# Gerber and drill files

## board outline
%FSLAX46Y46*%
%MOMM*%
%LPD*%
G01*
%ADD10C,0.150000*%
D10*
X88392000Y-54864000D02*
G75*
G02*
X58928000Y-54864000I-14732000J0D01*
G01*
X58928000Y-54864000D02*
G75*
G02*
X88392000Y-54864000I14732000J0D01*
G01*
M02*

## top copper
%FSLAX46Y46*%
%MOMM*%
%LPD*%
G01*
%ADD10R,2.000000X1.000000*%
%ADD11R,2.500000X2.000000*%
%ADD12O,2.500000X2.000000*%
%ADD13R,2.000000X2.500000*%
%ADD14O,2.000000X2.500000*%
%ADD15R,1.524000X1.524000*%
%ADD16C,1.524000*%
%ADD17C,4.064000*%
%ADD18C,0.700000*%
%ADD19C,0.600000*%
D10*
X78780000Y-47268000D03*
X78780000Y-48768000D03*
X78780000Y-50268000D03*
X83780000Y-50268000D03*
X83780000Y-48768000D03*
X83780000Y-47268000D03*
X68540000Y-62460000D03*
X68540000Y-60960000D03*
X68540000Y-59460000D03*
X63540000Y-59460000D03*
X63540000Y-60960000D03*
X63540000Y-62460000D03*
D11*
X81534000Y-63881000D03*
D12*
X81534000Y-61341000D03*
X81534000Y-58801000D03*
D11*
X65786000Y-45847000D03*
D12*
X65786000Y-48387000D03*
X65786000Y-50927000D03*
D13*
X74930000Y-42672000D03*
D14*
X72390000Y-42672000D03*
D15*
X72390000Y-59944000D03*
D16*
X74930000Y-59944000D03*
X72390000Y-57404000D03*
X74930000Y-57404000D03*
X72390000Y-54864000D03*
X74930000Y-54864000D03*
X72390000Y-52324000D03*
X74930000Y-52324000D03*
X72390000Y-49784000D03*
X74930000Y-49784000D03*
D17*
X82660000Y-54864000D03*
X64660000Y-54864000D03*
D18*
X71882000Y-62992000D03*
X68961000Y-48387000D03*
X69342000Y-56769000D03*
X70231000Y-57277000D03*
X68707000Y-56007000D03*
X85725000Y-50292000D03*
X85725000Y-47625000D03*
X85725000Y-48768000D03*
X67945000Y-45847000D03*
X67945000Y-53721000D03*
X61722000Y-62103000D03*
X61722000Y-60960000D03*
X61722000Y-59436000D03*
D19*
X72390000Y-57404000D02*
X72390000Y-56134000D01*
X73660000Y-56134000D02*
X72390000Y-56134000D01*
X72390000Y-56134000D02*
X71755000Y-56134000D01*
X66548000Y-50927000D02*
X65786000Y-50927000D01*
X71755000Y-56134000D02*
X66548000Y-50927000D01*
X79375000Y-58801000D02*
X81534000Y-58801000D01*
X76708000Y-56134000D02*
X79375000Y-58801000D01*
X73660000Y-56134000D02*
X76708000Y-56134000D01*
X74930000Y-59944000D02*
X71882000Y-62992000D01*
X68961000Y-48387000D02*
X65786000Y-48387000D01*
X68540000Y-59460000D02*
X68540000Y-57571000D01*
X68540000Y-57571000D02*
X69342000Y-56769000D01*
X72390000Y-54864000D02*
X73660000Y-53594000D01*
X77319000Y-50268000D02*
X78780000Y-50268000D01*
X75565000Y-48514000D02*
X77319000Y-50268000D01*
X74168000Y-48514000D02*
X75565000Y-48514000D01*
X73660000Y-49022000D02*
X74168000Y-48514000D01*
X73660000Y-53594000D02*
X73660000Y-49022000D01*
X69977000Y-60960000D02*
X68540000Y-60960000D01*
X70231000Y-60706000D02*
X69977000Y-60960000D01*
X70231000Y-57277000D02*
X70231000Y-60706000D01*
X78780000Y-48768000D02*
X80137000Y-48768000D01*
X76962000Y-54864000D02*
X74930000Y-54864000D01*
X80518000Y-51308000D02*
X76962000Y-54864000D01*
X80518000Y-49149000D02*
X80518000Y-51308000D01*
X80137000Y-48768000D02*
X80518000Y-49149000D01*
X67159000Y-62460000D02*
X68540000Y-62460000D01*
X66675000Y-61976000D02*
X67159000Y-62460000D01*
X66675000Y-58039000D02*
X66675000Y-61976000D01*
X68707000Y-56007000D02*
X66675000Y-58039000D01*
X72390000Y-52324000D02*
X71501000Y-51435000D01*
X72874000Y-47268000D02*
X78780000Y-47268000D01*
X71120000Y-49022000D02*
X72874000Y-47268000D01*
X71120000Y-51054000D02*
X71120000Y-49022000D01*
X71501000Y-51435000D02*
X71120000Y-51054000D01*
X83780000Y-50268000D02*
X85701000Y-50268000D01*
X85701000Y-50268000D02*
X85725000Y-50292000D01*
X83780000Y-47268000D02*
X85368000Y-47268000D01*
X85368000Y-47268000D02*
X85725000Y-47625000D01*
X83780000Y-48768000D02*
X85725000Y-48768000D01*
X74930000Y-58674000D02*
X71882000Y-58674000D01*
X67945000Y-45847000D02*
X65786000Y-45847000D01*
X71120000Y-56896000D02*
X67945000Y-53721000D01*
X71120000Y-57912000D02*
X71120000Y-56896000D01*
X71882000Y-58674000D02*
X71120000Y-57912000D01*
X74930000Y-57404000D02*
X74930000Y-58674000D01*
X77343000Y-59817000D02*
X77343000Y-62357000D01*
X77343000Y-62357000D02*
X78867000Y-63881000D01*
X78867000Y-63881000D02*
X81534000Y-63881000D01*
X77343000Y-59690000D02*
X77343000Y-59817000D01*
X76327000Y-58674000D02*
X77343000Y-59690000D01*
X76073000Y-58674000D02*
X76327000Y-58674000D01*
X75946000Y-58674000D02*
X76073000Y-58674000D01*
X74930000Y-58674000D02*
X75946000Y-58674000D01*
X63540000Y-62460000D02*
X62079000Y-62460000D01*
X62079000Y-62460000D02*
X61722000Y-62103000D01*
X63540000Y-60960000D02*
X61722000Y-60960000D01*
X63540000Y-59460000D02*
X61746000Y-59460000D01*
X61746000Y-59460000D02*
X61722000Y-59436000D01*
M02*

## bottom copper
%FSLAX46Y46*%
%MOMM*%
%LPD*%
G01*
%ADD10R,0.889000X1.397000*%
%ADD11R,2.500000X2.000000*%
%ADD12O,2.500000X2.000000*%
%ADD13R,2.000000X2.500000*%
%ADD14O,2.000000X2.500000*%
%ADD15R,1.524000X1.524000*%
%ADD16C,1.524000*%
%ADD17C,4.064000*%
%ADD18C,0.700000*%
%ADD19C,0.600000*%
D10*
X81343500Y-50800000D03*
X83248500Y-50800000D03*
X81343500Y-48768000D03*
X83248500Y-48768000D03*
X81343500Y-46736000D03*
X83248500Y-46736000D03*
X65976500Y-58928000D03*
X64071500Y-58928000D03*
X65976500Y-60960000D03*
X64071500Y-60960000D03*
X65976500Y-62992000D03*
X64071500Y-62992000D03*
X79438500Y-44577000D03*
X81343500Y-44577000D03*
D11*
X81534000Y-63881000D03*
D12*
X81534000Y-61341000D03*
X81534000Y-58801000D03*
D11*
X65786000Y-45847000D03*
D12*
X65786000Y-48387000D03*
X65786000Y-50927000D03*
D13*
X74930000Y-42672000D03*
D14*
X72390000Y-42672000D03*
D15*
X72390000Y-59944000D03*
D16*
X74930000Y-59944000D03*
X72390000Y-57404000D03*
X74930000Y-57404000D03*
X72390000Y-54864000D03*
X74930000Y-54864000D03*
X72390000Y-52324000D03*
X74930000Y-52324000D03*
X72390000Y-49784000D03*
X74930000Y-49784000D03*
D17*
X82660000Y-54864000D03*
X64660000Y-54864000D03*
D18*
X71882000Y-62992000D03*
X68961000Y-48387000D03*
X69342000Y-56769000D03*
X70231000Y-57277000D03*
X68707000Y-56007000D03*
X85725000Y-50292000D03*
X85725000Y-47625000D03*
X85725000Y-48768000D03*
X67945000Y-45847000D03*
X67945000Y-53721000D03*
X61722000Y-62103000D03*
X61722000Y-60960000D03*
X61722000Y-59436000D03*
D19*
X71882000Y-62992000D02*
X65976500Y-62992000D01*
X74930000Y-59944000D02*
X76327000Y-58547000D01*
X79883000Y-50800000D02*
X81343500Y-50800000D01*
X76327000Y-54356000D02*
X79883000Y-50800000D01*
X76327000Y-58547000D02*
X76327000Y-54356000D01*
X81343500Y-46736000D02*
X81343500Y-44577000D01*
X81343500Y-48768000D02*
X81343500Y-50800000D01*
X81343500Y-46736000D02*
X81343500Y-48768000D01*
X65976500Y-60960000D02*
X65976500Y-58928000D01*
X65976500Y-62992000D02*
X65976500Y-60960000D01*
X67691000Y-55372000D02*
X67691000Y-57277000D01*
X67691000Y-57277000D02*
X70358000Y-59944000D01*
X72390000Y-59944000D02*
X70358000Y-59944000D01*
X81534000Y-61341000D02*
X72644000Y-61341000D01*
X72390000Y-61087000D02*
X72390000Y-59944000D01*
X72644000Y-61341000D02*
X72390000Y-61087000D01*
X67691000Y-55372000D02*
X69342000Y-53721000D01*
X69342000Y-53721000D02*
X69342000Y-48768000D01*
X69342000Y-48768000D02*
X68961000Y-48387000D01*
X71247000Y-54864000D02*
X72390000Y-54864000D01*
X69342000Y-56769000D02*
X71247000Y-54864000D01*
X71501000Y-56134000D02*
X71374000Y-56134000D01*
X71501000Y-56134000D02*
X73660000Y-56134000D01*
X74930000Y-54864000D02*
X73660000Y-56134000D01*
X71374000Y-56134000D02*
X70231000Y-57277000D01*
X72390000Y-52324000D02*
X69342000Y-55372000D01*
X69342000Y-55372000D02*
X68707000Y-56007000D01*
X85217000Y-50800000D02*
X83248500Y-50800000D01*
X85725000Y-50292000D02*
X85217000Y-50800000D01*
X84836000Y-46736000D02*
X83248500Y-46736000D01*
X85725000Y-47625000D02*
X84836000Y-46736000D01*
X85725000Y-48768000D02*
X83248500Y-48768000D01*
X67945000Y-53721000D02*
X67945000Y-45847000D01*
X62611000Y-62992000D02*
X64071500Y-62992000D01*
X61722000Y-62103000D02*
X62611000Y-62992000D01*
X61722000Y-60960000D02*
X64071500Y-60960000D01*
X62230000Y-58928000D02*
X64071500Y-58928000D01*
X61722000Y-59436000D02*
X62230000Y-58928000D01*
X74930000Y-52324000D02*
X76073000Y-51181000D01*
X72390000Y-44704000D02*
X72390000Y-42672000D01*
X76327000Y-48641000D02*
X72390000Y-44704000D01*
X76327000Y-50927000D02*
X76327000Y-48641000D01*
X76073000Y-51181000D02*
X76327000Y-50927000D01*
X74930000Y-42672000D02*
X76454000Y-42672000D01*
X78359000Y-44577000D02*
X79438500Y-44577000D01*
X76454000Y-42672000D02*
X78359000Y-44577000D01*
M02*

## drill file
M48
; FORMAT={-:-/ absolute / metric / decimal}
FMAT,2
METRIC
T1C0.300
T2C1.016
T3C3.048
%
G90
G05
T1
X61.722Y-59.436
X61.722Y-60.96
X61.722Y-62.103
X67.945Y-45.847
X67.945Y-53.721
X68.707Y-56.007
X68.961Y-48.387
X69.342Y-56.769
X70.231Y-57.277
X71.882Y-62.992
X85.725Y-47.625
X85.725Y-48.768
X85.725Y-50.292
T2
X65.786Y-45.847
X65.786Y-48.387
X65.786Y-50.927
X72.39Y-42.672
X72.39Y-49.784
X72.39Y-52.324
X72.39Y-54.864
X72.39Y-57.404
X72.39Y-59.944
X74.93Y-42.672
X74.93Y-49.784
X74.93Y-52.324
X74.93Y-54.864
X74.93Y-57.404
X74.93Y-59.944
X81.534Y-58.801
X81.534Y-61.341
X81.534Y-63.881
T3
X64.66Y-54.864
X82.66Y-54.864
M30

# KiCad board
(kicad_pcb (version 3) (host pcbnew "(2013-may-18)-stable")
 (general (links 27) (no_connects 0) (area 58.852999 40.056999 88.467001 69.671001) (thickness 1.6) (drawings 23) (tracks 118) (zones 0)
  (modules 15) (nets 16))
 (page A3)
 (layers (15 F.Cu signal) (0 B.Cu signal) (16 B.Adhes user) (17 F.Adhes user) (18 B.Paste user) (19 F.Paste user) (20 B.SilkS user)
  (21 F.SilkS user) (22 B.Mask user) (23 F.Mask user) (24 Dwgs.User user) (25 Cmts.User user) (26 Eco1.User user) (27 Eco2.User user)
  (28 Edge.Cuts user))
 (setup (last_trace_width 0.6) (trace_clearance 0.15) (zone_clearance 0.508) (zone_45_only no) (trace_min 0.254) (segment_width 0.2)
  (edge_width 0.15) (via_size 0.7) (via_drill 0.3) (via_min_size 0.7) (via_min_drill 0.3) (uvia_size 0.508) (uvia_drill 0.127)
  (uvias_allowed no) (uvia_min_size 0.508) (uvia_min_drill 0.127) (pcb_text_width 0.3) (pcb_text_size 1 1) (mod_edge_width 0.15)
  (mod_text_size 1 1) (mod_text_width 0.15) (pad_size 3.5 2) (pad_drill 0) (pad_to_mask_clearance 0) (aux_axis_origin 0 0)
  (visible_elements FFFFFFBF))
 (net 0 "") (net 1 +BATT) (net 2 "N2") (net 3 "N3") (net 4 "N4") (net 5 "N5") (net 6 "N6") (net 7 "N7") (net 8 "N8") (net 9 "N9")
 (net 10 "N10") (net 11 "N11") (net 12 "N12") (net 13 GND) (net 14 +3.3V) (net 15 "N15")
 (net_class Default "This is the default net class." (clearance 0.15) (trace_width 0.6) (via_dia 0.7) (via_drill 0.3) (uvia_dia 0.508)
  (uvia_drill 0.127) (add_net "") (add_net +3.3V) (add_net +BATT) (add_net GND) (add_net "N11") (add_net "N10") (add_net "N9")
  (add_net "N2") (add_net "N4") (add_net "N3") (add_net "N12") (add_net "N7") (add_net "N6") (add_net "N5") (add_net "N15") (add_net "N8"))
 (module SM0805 (layer B.Cu) (at 82.296 50.8)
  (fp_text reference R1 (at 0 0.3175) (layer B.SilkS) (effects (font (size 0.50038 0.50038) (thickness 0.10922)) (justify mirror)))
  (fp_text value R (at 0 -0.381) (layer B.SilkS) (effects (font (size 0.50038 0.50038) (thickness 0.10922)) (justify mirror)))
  (pad 1 smd rect (at -0.9525 0) (size 0.889 1.397) (layers B.Cu B.Paste B.Mask) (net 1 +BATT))
  (pad 2 smd rect (at 0.9525 0) (size 0.889 1.397) (layers B.Cu B.Paste B.Mask) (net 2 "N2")))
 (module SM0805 (layer B.Cu) (at 82.296 48.768)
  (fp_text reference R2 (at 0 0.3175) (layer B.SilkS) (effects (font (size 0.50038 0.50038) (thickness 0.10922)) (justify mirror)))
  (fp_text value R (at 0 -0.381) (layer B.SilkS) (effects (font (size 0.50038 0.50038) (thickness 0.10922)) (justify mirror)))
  (pad 1 smd rect (at -0.9525 0) (size 0.889 1.397) (layers B.Cu B.Paste B.Mask) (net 1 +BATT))
  (pad 2 smd rect (at 0.9525 0) (size 0.889 1.397) (layers B.Cu B.Paste B.Mask) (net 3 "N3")))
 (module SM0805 (layer B.Cu) (at 82.296 46.736)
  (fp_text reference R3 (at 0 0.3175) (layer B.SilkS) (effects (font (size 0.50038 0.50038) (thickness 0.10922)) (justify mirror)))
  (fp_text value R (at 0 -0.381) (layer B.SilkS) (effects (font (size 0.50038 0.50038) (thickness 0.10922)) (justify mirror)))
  (pad 1 smd rect (at -0.9525 0) (size 0.889 1.397) (layers B.Cu B.Paste B.Mask) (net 1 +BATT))
  (pad 2 smd rect (at 0.9525 0) (size 0.889 1.397) (layers B.Cu B.Paste B.Mask) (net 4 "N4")))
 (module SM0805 (layer B.Cu) (at 65.024 58.928 180)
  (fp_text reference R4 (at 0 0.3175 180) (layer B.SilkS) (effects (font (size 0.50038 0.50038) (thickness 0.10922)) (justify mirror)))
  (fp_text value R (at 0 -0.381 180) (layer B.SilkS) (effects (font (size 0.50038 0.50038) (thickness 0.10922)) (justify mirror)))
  (pad 1 smd rect (at -0.9525 0 180) (size 0.889 1.397) (layers B.Cu B.Paste B.Mask) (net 1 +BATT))
  (pad 2 smd rect (at 0.9525 0 180) (size 0.889 1.397) (layers B.Cu B.Paste B.Mask) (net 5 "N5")))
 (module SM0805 (layer B.Cu) (at 65.024 60.96 180)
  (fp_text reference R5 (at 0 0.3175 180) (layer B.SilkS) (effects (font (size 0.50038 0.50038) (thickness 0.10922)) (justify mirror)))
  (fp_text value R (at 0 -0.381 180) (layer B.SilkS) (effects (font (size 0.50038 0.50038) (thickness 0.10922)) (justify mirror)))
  (pad 1 smd rect (at -0.9525 0 180) (size 0.889 1.397) (layers B.Cu B.Paste B.Mask) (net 1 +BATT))
  (pad 2 smd rect (at 0.9525 0 180) (size 0.889 1.397) (layers B.Cu B.Paste B.Mask) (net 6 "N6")))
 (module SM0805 (layer B.Cu) (at 65.024 62.992 180)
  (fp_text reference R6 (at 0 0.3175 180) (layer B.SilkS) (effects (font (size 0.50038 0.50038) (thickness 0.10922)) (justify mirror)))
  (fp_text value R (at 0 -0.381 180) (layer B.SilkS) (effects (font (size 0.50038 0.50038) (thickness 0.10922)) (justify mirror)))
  (pad 1 smd rect (at -0.9525 0 180) (size 0.889 1.397) (layers B.Cu B.Paste B.Mask) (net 1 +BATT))
  (pad 2 smd rect (at 0.9525 0 180) (size 0.889 1.397) (layers B.Cu B.Paste B.Mask) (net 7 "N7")))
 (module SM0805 (layer B.Cu) (at 80.391 44.577)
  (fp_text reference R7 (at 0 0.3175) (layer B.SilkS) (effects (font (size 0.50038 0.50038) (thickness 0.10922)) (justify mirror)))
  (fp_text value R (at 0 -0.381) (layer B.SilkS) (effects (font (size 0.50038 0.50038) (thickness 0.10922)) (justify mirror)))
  (pad 1 smd rect (at -0.9525 0) (size 0.889 1.397) (layers B.Cu B.Paste B.Mask) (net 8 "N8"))
  (pad 2 smd rect (at 0.9525 0) (size 0.889 1.397) (layers B.Cu B.Paste B.Mask) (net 1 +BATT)))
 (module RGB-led (layer F.Cu) (at 81.28 48.768 180)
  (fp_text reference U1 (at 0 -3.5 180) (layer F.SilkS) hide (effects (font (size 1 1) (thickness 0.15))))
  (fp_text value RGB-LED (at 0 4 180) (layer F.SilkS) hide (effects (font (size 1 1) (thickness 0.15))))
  (pad 1 smd rect (at 2.5 1.5 180) (size 2 1) (layers F.Cu F.Paste F.Mask) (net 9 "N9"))
  (pad 2 smd rect (at 2.5 0 180) (size 2 1) (layers F.Cu F.Paste F.Mask) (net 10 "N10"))
  (pad 3 smd rect (at 2.5 -1.5 180) (size 2 1) (layers F.Cu F.Paste F.Mask) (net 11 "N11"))
  (pad 4 smd rect (at -2.5 -1.5 180) (size 2 1) (layers F.Cu F.Paste F.Mask) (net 2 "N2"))
  (pad 5 smd rect (at -2.5 0 180) (size 2 1) (layers F.Cu F.Paste F.Mask) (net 3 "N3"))
  (pad 6 smd rect (at -2.5 1.5 180) (size 2 1) (layers F.Cu F.Paste F.Mask) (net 4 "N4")))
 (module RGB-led (layer F.Cu) (at 66.04 60.96)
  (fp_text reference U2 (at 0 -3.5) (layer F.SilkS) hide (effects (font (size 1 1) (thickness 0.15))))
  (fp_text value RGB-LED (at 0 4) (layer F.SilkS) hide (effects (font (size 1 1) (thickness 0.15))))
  (pad 1 smd rect (at 2.5 1.5) (size 2 1) (layers F.Cu F.Paste F.Mask) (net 9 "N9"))
  (pad 2 smd rect (at 2.5 0) (size 2 1) (layers F.Cu F.Paste F.Mask) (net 10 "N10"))
  (pad 3 smd rect (at 2.5 -1.5) (size 2 1) (layers F.Cu F.Paste F.Mask) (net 11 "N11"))
  (pad 4 smd rect (at -2.5 -1.5) (size 2 1) (layers F.Cu F.Paste F.Mask) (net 5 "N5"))
  (pad 5 smd rect (at -2.5 0) (size 2 1) (layers F.Cu F.Paste F.Mask) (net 6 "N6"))
  (pad 6 smd rect (at -2.5 1.5) (size 2 1) (layers F.Cu F.Paste F.Mask) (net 7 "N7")))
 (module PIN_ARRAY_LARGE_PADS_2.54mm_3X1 (layer F.Cu) (at 81.534 61.341 90)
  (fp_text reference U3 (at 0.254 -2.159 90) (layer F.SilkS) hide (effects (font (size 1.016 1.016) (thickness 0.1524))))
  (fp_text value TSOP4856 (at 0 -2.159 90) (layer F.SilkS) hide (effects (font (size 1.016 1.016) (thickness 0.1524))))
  (pad 1 thru_hole rect (at -2.54 0 90) (size 2 2.5) (drill 1.016) (layers *.Cu *.Mask F.SilkS) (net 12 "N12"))
  (pad 2 thru_hole oval (at 0 0 90) (size 2 2.5) (drill 1.016) (layers *.Cu *.Mask F.SilkS) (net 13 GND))
  (pad 3 thru_hole oval (at 2.54 0 90) (size 2 2.5) (drill 1.016) (layers *.Cu *.Mask F.SilkS) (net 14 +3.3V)))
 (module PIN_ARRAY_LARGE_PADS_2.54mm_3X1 (layer F.Cu) (at 65.786 48.387 270)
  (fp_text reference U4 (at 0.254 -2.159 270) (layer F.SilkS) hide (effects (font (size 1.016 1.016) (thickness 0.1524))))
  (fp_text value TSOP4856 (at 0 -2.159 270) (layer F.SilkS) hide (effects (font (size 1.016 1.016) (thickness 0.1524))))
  (pad 1 thru_hole rect (at -2.54 0 270) (size 2 2.5) (drill 1.016) (layers *.Cu *.Mask F.SilkS) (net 12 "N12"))
  (pad 2 thru_hole oval (at 0 0 270) (size 2 2.5) (drill 1.016) (layers *.Cu *.Mask F.SilkS) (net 13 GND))
  (pad 3 thru_hole oval (at 2.54 0 270) (size 2 2.5) (drill 1.016) (layers *.Cu *.Mask F.SilkS) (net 14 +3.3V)))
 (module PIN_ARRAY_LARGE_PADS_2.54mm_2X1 (layer F.Cu) (at 73.66 42.672 180)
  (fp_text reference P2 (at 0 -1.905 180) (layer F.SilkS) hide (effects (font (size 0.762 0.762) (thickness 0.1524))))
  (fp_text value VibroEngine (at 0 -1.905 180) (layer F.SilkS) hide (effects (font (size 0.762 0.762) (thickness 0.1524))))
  (pad 1 thru_hole rect (at -1.27 0 180) (size 2 2.5) (drill 1.016) (layers *.Cu *.Mask F.SilkS) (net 8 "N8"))
  (pad 2 thru_hole oval (at 1.27 0 180) (size 2 2.5) (drill 1.016) (layers *.Cu *.Mask F.SilkS) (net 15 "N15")))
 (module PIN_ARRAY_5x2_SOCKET (layer B.Cu) (at 73.66 54.864 90)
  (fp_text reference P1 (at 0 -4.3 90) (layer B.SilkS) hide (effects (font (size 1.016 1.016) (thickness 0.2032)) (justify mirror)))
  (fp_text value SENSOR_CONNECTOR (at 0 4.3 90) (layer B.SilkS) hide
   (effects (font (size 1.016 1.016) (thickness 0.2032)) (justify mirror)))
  (pad 1 thru_hole rect (at -5.08 -1.27 90) (size 1.524 1.524) (drill 1.016) (layers *.Cu *.Mask B.SilkS) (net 13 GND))
  (pad 2 thru_hole circle (at -5.08 1.27 90) (size 1.524 1.524) (drill 1.016) (layers *.Cu *.Mask B.SilkS) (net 1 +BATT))
  (pad 3 thru_hole circle (at -2.54 -1.27 90) (size 1.524 1.524) (drill 1.016) (layers *.Cu *.Mask B.SilkS) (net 14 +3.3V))
  (pad 4 thru_hole circle (at -2.54 1.27 90) (size 1.524 1.524) (drill 1.016) (layers *.Cu *.Mask B.SilkS) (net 12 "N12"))
  (pad 5 thru_hole circle (at 0 -1.27 90) (size 1.524 1.524) (drill 1.016) (layers *.Cu *.Mask B.SilkS) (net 11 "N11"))
  (pad 6 thru_hole circle (at 0 1.27 90) (size 1.524 1.524) (drill 1.016) (layers *.Cu *.Mask B.SilkS) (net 10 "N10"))
  (pad 7 thru_hole circle (at 2.54 -1.27 90) (size 1.524 1.524) (drill 1.016) (layers *.Cu *.Mask B.SilkS) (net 9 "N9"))
  (pad 8 thru_hole circle (at 2.54 1.27 90) (size 1.524 1.524) (drill 1.016) (layers *.Cu *.Mask B.SilkS) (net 15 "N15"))
  (pad 9 thru_hole circle (at 5.08 -1.27 90) (size 1.524 1.524) (drill 1.016) (layers *.Cu *.Mask B.SilkS))
  (pad 10 thru_hole circle (at 5.08 1.27 90) (size 1.524 1.524) (drill 1.016) (layers *.Cu *.Mask B.SilkS)))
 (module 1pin (layer F.Cu) (at 82.66 54.864)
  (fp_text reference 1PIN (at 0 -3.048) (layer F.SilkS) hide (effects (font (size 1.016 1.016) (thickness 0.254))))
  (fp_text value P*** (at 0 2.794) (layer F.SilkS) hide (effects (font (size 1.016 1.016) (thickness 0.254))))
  (pad 1 thru_hole circle (at 0 0) (size 4.064 4.064) (drill 3.048) (layers *.Cu *.Mask F.SilkS)))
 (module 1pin (layer F.Cu) (at 64.66 54.864)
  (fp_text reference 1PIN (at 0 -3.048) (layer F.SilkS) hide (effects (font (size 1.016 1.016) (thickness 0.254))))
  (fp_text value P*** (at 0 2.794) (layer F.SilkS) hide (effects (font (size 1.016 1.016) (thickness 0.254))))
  (pad 1 thru_hole circle (at 0 0) (size 4.064 4.064) (drill 3.048) (layers *.Cu *.Mask F.SilkS)))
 (gr_circle (center 73.66 54.864) (end 88.392 54.864) (layer Edge.Cuts) (width 0.15))
 (segment (start 72.39 57.404) (end 72.39 56.134) (width 0.6) (layer F.Cu) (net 14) (status 400000))
 (segment (start 73.66 56.134) (end 72.39 56.134) (width 0.6) (layer F.Cu) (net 14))
 (segment (start 72.39 56.134) (end 71.755 56.134) (width 0.6) (layer F.Cu) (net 14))
 (segment (start 66.548 50.927) (end 65.786 50.927) (width 0.6) (layer F.Cu) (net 14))
 (segment (start 71.755 56.134) (end 66.548 50.927) (width 0.6) (layer F.Cu) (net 14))
 (segment (start 79.375 58.801) (end 81.534 58.801) (width 0.6) (layer F.Cu) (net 14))
 (segment (start 76.708 56.134) (end 79.375 58.801) (width 0.6) (layer F.Cu) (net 14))
 (segment (start 73.66 56.134) (end 76.708 56.134) (width 0.6) (layer F.Cu) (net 14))
 (segment (start 74.93 59.944) (end 71.882 62.992) (width 0.6) (layer F.Cu) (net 1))
 (segment (start 71.882 62.992) (end 65.9765 62.992) (width 0.6) (layer B.Cu) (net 1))
 (via (at 71.882 62.992) (size 0.7) (layers F.Cu B.Cu) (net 1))
 (segment (start 74.93 59.944) (end 76.327 58.547) (width 0.6) (layer B.Cu) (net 1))
 (segment (start 79.883 50.8) (end 81.3435 50.8) (width 0.6) (layer B.Cu) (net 1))
 (segment (start 76.327 54.356) (end 79.883 50.8) (width 0.6) (layer B.Cu) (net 1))
 (segment (start 76.327 58.547) (end 76.327 54.356) (width 0.6) (layer B.Cu) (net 1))
 (segment (start 81.3435 46.736) (end 81.3435 44.577) (width 0.6) (layer B.Cu) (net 1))
 (segment (start 81.3435 48.768) (end 81.3435 50.8) (width 0.6) (layer B.Cu) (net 1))
 (segment (start 81.3435 46.736) (end 81.3435 48.768) (width 0.6) (layer B.Cu) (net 1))
 (segment (start 65.9765 60.96) (end 65.9765 58.928) (width 0.6) (layer B.Cu) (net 1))
 (segment (start 65.9765 62.992) (end 65.9765 60.96) (width 0.6) (layer B.Cu) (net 1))
 (segment (start 67.691 55.372) (end 67.691 57.277) (width 0.6) (layer B.Cu) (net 13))
 (segment (start 67.691 57.277) (end 70.358 59.944) (width 0.6) (layer B.Cu) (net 13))
 (segment (start 72.39 59.944) (end 70.358 59.944) (width 0.6) (layer B.Cu) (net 13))
 (segment (start 68.961 48.387) (end 65.786 48.387) (width 0.6) (layer F.Cu) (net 13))
 (segment (start 81.534 61.341) (end 72.644 61.341) (width 0.6) (layer B.Cu) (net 13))
 (segment (start 72.39 61.087) (end 72.39 59.944) (width 0.6) (layer B.Cu) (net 13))
 (segment (start 72.644 61.341) (end 72.39 61.087) (width 0.6) (layer B.Cu) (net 13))
 (segment (start 67.691 55.372) (end 69.342 53.721) (width 0.6) (layer B.Cu) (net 13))
 (segment (start 69.342 53.721) (end 69.342 48.768) (width 0.6) (layer B.Cu) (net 13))
 (via (at 68.961 48.387) (size 0.7) (layers F.Cu B.Cu) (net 13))
 (segment (start 69.342 48.768) (end 68.961 48.387) (width 0.6) (layer B.Cu) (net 13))
 (segment (start 68.54 59.46) (end 68.54 57.571) (width 0.6) (layer F.Cu) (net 11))
 (segment (start 71.247 54.864) (end 72.39 54.864) (width 0.6) (layer B.Cu) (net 11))
 (segment (start 69.342 56.769) (end 71.247 54.864) (width 0.6) (layer B.Cu) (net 11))
 (via (at 69.342 56.769) (size 0.7) (layers F.Cu B.Cu) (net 11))
 (segment (start 68.54 57.571) (end 69.342 56.769) (width 0.6) (layer F.Cu) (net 11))
 (segment (start 72.39 54.864) (end 73.66 53.594) (width 0.6) (layer F.Cu) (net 11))
 (segment (start 77.319 50.268) (end 78.78 50.268) (width 0.6) (layer F.Cu) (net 11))
 (segment (start 75.565 48.514) (end 77.319 50.268) (width 0.6) (layer F.Cu) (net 11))
 (segment (start 74.168 48.514) (end 75.565 48.514) (width 0.6) (layer F.Cu) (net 11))
 (segment (start 73.66 49.022) (end 74.168 48.514) (width 0.6) (layer F.Cu) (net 11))
 (segment (start 73.66 53.594) (end 73.66 49.022) (width 0.6) (layer F.Cu) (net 11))
 (segment (start 71.501 56.134) (end 71.374 56.134) (width 0.6) (layer B.Cu) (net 10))
 (segment (start 71.501 56.134) (end 73.66 56.134) (width 0.6) (layer B.Cu) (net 10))
 (segment (start 74.93 54.864) (end 73.66 56.134) (width 0.6) (layer B.Cu) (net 10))
 (segment (start 69.977 60.96) (end 68.54 60.96) (width 0.6) (layer F.Cu) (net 10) (status 800000))
 (segment (start 70.231 60.706) (end 69.977 60.96) (width 0.6) (layer F.Cu) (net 10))
 (segment (start 70.231 57.277) (end 70.231 60.706) (width 0.6) (layer F.Cu) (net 10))
 (via (at 70.231 57.277) (size 0.7) (layers F.Cu B.Cu) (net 10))
 (segment (start 71.374 56.134) (end 70.231 57.277) (width 0.6) (layer B.Cu) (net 10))
 (segment (start 78.78 48.768) (end 80.137 48.768) (width 0.6) (layer F.Cu) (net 10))
 (segment (start 76.962 54.864) (end 74.93 54.864) (width 0.6) (layer F.Cu) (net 10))
 (segment (start 80.518 51.308) (end 76.962 54.864) (width 0.6) (layer F.Cu) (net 10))
 (segment (start 80.518 49.149) (end 80.518 51.308) (width 0.6) (layer F.Cu) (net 10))
 (segment (start 80.137 48.768) (end 80.518 49.149) (width 0.6) (layer F.Cu) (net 10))
 (segment (start 72.39 52.324) (end 69.342 55.372) (width 0.6) (layer B.Cu) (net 9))
 (segment (start 67.159 62.46) (end 68.54 62.46) (width 0.6) (layer F.Cu) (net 9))
 (segment (start 66.675 61.976) (end 67.159 62.46) (width 0.6) (layer F.Cu) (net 9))
 (segment (start 66.675 58.039) (end 66.675 61.976) (width 0.6) (layer F.Cu) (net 9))
 (segment (start 68.707 56.007) (end 66.675 58.039) (width 0.6) (layer F.Cu) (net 9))
 (via (at 68.707 56.007) (size 0.7) (layers F.Cu B.Cu) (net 9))
 (segment (start 69.342 55.372) (end 68.707 56.007) (width 0.6) (layer B.Cu) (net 9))
 (segment (start 72.39 52.324) (end 71.501 51.435) (width 0.6) (layer F.Cu) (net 9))
 (segment (start 72.874 47.268) (end 78.78 47.268) (width 0.6) (layer F.Cu) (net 9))
 (segment (start 71.12 49.022) (end 72.874 47.268) (width 0.6) (layer F.Cu) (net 9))
 (segment (start 71.12 51.054) (end 71.12 49.022) (width 0.6) (layer F.Cu) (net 9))
 (segment (start 71.501 51.435) (end 71.12 51.054) (width 0.6) (layer F.Cu) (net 9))
 (segment (start 83.78 50.268) (end 85.701 50.268) (width 0.6) (layer F.Cu) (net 2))
 (segment (start 85.217 50.8) (end 83.2485 50.8) (width 0.6) (layer B.Cu) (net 2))
 (segment (start 85.725 50.292) (end 85.217 50.8) (width 0.6) (layer B.Cu) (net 2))
 (via (at 85.725 50.292) (size 0.7) (layers F.Cu B.Cu) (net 2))
 (segment (start 85.701 50.268) (end 85.725 50.292) (width 0.6) (layer F.Cu) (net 2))
 (segment (start 83.78 47.268) (end 85.368 47.268) (width 0.6) (layer F.Cu) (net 4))
 (segment (start 84.836 46.736) (end 83.2485 46.736) (width 0.6) (layer B.Cu) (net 4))
 (segment (start 85.725 47.625) (end 84.836 46.736) (width 0.6) (layer B.Cu) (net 4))
 (via (at 85.725 47.625) (size 0.7) (layers F.Cu B.Cu) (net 4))
 (segment (start 85.368 47.268) (end 85.725 47.625) (width 0.6) (layer F.Cu) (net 4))
 (segment (start 83.78 48.768) (end 85.725 48.768) (width 0.6) (layer F.Cu) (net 3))
 (segment (start 85.725 48.768) (end 83.2485 48.768) (width 0.6) (layer B.Cu) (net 3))
 (via (at 85.725 48.768) (size 0.7) (layers F.Cu B.Cu) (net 3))
 (segment (start 74.93 58.674) (end 71.882 58.674) (width 0.6) (layer F.Cu) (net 12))
 (segment (start 67.945 45.847) (end 65.786 45.847) (width 0.6) (layer F.Cu) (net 12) (status 800000))
 (via (at 67.945 45.847) (size 0.7) (layers F.Cu B.Cu) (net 12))
 (segment (start 67.945 53.721) (end 67.945 45.847) (width 0.6) (layer B.Cu) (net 12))
 (via (at 67.945 53.721) (size 0.7) (layers F.Cu B.Cu) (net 12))
 (segment (start 71.12 56.896) (end 67.945 53.721) (width 0.6) (layer F.Cu) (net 12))
 (segment (start 71.12 57.912) (end 71.12 56.896) (width 0.6) (layer F.Cu) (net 12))
 (segment (start 71.882 58.674) (end 71.12 57.912) (width 0.6) (layer F.Cu) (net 12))
 (segment (start 74.93 57.404) (end 74.93 58.674) (width 0.6) (layer F.Cu) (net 12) (status 400000))
 (segment (start 77.343 59.817) (end 77.343 62.357) (width 0.6) (layer F.Cu) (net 12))
 (segment (start 77.343 62.357) (end 78.867 63.881) (width 0.6) (layer F.Cu) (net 12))
 (segment (start 78.867 63.881) (end 81.534 63.881) (width 0.6) (layer F.Cu) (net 12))
 (segment (start 77.343 59.69) (end 77.343 59.817) (width 0.6) (layer F.Cu) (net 12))
 (segment (start 76.327 58.674) (end 77.343 59.69) (width 0.6) (layer F.Cu) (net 12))
 (segment (start 76.073 58.674) (end 76.327 58.674) (width 0.6) (layer F.Cu) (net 12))
 (segment (start 75.946 58.674) (end 76.073 58.674) (width 0.6) (layer F.Cu) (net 12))
 (segment (start 74.93 58.674) (end 75.946 58.674) (width 0.6) (layer F.Cu) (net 12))
 (segment (start 63.54 62.46) (end 62.079 62.46) (width 0.6) (layer F.Cu) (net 7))
 (segment (start 62.611 62.992) (end 64.0715 62.992) (width 0.6) (layer B.Cu) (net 7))
 (segment (start 61.722 62.103) (end 62.611 62.992) (width 0.6) (layer B.Cu) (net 7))
 (via (at 61.722 62.103) (size 0.7) (layers F.Cu B.Cu) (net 7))
 (segment (start 62.079 62.46) (end 61.722 62.103) (width 0.6) (layer F.Cu) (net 7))
 (segment (start 63.54 60.96) (end 61.722 60.96) (width 0.6) (layer F.Cu) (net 6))
 (segment (start 61.722 60.96) (end 64.0715 60.96) (width 0.6) (layer B.Cu) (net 6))
 (via (at 61.722 60.96) (size 0.7) (layers F.Cu B.Cu) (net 6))
 (segment (start 63.54 59.46) (end 61.746 59.46) (width 0.6) (layer F.Cu) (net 5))
 (segment (start 62.23 58.928) (end 64.0715 58.928) (width 0.6) (layer B.Cu) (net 5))
 (segment (start 61.722 59.436) (end 62.23 58.928) (width 0.6) (layer B.Cu) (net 5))
 (via (at 61.722 59.436) (size 0.7) (layers F.Cu B.Cu) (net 5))
 (segment (start 61.746 59.46) (end 61.722 59.436) (width 0.6) (layer F.Cu) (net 5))
 (segment (start 74.93 52.324) (end 76.073 51.181) (width 0.6) (layer B.Cu) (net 15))
 (segment (start 72.39 44.704) (end 72.39 42.672) (width 0.6) (layer B.Cu) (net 15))
 (segment (start 76.327 48.641) (end 72.39 44.704) (width 0.6) (layer B.Cu) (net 15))
 (segment (start 76.327 50.927) (end 76.327 48.641) (width 0.6) (layer B.Cu) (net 15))
 (segment (start 76.073 51.181) (end 76.327 50.927) (width 0.6) (layer B.Cu) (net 15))
 (segment (start 74.93 42.672) (end 76.454 42.672) (width 0.6) (layer B.Cu) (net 8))
 (segment (start 78.359 44.577) (end 79.4385 44.577) (width 0.6) (layer B.Cu) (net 8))
 (segment (start 76.454 42.672) (end 78.359 44.577) (width 0.6) (layer B.Cu) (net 8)))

